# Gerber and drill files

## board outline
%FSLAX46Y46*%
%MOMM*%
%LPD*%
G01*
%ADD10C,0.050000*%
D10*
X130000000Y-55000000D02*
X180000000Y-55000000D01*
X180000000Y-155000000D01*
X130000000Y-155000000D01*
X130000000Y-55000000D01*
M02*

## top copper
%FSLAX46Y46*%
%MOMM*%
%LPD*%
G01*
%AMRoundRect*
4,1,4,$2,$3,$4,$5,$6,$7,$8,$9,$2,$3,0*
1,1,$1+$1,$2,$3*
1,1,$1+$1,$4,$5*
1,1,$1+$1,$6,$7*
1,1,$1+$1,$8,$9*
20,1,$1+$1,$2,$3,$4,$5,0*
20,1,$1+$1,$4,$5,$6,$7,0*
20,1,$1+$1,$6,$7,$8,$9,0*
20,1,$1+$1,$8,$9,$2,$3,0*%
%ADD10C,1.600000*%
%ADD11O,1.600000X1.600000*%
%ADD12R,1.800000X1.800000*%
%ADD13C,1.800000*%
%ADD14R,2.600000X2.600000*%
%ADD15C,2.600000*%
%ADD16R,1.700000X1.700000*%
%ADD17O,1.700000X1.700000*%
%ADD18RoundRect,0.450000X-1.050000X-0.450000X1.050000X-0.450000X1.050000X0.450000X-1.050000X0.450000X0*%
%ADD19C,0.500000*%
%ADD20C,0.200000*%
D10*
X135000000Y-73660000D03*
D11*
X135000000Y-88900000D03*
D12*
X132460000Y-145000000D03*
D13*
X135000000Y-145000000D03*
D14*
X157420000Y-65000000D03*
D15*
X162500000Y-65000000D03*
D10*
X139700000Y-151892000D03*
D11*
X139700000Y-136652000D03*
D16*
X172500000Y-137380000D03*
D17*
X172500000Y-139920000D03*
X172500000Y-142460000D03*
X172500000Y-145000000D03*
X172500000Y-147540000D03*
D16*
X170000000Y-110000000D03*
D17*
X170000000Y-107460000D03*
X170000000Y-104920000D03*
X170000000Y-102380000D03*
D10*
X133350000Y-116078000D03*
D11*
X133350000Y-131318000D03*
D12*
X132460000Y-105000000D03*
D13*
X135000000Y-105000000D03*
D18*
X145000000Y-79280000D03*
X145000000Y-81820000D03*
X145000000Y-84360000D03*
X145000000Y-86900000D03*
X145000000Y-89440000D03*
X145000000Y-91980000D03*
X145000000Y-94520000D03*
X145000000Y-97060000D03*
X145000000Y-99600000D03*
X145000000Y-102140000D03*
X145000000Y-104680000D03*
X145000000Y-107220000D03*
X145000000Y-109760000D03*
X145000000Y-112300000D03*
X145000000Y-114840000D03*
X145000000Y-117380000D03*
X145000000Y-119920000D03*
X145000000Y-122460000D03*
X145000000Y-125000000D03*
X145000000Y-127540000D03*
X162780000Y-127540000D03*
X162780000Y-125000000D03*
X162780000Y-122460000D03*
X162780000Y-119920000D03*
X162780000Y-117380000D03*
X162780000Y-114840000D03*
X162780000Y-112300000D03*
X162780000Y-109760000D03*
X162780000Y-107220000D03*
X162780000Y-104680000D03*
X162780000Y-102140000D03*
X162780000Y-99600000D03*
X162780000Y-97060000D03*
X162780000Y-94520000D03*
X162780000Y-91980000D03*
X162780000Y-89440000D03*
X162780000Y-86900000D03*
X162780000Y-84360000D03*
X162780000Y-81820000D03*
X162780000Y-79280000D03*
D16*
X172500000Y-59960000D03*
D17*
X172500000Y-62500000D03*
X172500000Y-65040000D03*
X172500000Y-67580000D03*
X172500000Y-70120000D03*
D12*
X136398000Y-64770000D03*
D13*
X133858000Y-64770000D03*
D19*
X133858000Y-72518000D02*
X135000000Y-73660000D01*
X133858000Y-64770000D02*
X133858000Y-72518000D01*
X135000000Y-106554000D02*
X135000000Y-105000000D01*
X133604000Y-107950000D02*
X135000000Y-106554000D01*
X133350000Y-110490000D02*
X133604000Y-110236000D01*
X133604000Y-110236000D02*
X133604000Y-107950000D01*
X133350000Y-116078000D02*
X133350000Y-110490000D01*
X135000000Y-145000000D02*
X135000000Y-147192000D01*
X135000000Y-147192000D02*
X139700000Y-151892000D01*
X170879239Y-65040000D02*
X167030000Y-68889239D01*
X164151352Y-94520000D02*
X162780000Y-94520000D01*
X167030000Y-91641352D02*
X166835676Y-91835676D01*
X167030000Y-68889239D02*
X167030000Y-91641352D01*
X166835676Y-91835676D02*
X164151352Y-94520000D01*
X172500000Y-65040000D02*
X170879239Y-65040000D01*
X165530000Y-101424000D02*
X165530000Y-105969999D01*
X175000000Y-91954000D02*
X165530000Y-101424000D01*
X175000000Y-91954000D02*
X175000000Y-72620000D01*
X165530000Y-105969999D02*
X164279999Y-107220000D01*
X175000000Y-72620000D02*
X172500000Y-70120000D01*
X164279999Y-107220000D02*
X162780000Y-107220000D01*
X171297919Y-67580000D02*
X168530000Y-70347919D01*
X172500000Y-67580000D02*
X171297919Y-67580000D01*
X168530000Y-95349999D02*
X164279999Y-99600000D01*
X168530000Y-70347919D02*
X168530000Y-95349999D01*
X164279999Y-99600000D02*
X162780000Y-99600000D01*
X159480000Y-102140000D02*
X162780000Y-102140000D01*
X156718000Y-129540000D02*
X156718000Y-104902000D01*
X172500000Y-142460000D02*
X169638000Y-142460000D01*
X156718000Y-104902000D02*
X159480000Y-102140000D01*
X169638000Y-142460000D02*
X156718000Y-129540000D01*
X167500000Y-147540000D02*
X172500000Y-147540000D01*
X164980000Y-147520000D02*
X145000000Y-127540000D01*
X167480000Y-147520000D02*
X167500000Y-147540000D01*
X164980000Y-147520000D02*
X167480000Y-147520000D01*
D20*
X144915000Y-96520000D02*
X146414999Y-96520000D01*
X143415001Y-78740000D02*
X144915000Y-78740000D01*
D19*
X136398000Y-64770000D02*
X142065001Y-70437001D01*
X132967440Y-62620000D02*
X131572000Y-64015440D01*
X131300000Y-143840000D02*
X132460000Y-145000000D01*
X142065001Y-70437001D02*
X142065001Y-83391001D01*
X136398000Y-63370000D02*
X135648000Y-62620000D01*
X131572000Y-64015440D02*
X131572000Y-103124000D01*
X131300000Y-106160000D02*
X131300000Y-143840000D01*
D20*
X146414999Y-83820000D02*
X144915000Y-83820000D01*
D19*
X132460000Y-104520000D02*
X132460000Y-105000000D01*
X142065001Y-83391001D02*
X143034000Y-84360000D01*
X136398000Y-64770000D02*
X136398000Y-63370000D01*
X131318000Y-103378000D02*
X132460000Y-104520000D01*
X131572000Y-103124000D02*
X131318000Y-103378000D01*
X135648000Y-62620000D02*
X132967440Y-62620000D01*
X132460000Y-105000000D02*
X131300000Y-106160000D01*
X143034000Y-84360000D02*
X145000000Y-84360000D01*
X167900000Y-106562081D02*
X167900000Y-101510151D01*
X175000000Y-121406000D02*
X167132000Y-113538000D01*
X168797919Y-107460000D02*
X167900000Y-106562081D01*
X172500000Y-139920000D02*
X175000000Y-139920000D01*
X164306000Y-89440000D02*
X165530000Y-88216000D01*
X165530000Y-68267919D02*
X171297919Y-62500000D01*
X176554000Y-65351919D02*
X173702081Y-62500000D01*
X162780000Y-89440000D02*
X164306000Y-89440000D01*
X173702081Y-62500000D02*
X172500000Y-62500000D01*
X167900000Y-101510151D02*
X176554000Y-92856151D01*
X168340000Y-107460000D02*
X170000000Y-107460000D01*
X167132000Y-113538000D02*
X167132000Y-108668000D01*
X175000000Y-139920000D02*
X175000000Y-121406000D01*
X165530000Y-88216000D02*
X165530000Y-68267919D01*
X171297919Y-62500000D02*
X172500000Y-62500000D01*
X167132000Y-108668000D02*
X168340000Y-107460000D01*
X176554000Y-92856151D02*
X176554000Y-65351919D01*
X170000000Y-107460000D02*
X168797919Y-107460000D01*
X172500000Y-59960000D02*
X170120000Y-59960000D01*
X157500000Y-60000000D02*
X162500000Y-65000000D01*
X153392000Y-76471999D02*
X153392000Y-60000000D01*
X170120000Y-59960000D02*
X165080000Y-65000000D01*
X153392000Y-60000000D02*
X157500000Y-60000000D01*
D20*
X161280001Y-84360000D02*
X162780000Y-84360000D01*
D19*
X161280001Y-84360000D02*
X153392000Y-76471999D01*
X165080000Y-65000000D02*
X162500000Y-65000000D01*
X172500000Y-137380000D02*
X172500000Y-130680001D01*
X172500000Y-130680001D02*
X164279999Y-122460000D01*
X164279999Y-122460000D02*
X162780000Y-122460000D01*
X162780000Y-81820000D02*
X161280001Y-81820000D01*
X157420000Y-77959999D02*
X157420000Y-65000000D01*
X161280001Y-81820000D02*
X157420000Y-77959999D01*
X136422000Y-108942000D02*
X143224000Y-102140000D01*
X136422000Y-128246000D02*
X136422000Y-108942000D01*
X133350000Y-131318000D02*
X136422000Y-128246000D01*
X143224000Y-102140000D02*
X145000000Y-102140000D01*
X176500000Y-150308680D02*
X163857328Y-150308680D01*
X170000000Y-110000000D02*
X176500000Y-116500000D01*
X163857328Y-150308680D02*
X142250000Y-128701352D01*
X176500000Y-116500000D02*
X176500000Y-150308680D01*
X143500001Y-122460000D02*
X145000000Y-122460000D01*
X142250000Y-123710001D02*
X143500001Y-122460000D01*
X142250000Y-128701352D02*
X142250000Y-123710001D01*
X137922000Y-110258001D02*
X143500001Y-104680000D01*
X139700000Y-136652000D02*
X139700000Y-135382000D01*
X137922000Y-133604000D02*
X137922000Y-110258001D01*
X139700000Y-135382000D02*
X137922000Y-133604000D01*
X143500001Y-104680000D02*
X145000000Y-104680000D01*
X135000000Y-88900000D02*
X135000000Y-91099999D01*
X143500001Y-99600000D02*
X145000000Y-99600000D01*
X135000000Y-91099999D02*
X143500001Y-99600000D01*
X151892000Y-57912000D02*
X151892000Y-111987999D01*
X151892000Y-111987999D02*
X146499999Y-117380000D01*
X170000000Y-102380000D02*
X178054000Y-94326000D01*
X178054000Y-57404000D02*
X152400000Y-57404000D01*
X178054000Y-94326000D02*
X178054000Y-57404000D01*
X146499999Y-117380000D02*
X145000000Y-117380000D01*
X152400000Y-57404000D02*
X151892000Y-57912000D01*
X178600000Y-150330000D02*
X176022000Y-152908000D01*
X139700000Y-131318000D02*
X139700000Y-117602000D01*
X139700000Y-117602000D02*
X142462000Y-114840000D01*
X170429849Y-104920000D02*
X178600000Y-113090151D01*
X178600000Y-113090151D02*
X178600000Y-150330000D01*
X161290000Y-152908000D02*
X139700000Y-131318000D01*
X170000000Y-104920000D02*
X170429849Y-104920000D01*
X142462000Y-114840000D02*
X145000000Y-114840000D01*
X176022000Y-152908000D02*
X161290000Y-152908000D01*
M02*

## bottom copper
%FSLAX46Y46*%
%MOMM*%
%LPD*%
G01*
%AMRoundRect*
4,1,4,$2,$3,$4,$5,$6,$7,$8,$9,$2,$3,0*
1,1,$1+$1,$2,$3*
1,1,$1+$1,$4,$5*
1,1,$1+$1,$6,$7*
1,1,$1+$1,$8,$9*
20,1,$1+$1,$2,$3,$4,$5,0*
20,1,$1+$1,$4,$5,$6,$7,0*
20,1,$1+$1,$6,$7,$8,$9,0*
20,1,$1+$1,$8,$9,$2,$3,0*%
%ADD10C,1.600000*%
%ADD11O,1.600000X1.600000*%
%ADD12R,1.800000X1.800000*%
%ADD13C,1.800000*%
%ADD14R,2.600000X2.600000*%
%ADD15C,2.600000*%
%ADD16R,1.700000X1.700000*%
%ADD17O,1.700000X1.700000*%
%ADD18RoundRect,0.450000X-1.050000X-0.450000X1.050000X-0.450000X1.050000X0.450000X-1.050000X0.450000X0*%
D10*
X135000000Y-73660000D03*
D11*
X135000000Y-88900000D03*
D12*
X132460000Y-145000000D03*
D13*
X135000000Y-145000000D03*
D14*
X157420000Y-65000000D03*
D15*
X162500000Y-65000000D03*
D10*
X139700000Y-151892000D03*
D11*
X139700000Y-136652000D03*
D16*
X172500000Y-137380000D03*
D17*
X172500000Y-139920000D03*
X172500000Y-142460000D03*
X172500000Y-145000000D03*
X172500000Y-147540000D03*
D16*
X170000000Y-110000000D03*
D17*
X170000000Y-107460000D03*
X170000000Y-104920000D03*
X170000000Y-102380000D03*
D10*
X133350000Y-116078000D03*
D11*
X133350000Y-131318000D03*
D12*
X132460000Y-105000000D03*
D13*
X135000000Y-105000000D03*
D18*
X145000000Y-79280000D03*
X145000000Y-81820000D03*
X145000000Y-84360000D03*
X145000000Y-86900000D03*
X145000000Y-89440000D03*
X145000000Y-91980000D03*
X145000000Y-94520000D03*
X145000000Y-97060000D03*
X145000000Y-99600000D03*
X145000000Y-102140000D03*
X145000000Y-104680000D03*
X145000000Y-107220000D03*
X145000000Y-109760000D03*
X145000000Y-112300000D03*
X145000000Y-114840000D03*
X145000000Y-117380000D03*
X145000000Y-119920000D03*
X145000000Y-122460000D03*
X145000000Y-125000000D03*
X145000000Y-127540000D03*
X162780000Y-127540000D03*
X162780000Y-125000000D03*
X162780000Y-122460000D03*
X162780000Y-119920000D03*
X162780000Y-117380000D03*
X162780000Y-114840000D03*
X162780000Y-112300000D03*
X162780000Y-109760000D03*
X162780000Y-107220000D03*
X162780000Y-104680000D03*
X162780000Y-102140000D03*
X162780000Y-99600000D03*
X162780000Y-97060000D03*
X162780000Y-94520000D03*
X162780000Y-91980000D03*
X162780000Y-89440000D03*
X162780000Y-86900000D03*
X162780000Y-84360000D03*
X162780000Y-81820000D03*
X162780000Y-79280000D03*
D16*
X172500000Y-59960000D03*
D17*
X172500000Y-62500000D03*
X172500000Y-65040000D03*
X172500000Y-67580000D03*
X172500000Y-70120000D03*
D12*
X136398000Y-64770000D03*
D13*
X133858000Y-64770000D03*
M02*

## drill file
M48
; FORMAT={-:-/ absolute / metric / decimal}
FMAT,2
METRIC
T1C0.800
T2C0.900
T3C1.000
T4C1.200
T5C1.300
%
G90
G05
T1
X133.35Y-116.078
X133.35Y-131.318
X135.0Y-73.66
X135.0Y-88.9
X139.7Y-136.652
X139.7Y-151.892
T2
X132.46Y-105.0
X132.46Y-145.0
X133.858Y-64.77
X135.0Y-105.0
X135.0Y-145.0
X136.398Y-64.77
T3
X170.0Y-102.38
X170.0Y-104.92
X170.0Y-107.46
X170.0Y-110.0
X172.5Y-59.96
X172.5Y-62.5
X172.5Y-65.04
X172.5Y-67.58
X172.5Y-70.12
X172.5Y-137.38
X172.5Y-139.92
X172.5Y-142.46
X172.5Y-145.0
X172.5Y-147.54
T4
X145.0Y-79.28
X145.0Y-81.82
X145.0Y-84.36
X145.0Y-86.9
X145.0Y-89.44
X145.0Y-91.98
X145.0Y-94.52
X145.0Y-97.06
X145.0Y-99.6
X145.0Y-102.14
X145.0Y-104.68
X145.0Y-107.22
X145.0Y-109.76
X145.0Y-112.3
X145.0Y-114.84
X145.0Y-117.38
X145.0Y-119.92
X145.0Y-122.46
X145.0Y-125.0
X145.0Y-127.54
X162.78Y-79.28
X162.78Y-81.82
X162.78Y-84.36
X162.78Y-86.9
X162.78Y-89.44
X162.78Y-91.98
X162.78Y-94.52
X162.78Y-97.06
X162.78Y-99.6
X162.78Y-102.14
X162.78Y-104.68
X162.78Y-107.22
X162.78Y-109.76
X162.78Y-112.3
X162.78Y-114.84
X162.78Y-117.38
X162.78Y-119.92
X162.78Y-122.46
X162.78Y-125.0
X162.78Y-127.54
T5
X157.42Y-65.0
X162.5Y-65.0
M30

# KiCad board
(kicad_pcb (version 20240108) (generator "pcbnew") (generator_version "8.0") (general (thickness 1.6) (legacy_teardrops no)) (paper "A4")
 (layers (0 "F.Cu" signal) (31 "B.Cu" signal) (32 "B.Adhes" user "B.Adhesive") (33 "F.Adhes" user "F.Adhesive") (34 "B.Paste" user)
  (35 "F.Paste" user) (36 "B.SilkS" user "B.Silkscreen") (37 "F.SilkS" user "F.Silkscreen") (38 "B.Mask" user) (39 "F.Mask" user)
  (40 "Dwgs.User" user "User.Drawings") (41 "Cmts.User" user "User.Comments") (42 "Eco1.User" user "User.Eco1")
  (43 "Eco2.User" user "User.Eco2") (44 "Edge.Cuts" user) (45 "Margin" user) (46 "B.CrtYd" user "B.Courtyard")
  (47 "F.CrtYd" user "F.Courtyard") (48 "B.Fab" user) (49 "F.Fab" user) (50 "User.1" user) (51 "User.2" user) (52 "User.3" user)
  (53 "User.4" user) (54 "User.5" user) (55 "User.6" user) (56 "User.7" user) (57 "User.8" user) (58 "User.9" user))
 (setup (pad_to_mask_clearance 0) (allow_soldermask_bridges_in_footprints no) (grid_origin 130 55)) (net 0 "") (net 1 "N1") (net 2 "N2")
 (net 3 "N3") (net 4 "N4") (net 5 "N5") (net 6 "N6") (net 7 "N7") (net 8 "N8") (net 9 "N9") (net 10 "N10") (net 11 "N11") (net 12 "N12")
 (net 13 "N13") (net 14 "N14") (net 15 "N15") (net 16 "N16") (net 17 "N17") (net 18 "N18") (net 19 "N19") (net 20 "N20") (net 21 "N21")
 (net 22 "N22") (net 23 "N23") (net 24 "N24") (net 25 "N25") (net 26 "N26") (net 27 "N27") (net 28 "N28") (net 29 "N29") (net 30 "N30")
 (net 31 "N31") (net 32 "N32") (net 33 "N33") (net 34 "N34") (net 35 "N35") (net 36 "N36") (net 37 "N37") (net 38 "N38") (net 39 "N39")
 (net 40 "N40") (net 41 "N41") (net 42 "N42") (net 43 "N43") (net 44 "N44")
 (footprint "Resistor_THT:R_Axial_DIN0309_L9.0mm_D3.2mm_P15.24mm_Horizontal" (layer "F.Cu") (at 135 73.66 -90)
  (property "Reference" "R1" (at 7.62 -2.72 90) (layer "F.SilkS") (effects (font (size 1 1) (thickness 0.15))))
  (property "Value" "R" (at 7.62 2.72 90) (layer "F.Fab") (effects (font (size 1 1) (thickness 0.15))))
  (pad "1" thru_hole circle (at 0 0 270) (size 1.6 1.6) (drill 0.8) (layers "*.Cu" "*.Mask") (remove_unused_layers no) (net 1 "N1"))
  (pad "2" thru_hole oval (at 15.24 0 270) (size 1.6 1.6) (drill 0.8) (layers "*.Cu" "*.Mask") (remove_unused_layers no) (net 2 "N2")))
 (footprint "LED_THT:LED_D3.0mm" (layer "F.Cu") (at 132.46 145)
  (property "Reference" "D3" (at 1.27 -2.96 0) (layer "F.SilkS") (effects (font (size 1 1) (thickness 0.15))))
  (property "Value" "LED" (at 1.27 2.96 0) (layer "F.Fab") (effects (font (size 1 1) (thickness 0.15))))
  (pad "1" thru_hole rect (at 0 0) (size 1.8 1.8) (drill 0.9) (layers "*.Cu" "*.Mask") (remove_unused_layers no) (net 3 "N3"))
  (pad "2" thru_hole circle (at 2.54 0) (size 1.8 1.8) (drill 0.9) (layers "*.Cu" "*.Mask") (remove_unused_layers no) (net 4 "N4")))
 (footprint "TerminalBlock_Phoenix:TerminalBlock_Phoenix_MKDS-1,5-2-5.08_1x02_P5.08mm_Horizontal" (layer "F.Cu") (at 157.42 65)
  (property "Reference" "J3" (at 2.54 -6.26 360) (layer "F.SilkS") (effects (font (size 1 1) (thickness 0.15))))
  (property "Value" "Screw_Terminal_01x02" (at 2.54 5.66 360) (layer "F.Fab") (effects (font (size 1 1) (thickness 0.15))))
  (pad "1" thru_hole rect (at 0 0) (size 2.6 2.6) (drill 1.3) (layers "*.Cu" "*.Mask") (remove_unused_layers no) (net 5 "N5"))
  (pad "2" thru_hole circle (at 5.08 0) (size 2.6 2.6) (drill 1.3) (layers "*.Cu" "*.Mask") (remove_unused_layers no) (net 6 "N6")))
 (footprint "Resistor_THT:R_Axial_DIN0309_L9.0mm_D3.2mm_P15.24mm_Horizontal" (layer "F.Cu") (at 139.7 151.892 90)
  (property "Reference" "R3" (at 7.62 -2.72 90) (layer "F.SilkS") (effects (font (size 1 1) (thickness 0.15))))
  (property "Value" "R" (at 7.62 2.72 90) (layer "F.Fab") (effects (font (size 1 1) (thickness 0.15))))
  (pad "1" thru_hole circle (at 0 0 90) (size 1.6 1.6) (drill 0.8) (layers "*.Cu" "*.Mask") (remove_unused_layers no) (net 4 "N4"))
  (pad "2" thru_hole oval (at 15.24 0 90) (size 1.6 1.6) (drill 0.8) (layers "*.Cu" "*.Mask") (remove_unused_layers no) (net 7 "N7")))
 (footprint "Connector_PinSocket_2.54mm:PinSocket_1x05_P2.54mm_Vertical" (layer "F.Cu") (at 172.5 137.38)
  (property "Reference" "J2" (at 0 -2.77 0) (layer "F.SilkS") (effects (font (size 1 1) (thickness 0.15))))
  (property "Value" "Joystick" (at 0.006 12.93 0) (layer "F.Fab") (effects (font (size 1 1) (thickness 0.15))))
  (pad "1" thru_hole rect (at 0 0) (size 1.7 1.7) (drill 1) (layers "*.Cu" "*.Mask") (remove_unused_layers no) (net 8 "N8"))
  (pad "2" thru_hole oval (at 0 2.54) (size 1.7 1.7) (drill 1) (layers "*.Cu" "*.Mask") (remove_unused_layers no) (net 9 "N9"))
  (pad "3" thru_hole oval (at 0 5.08) (size 1.7 1.7) (drill 1) (layers "*.Cu" "*.Mask") (remove_unused_layers no) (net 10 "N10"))
  (pad "4" thru_hole oval (at 0 7.62) (size 1.7 1.7) (drill 1) (layers "*.Cu" "*.Mask") (remove_unused_layers no) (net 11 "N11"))
  (pad "5" thru_hole oval (at 0 10.16) (size 1.7 1.7) (drill 1) (layers "*.Cu" "*.Mask") (remove_unused_layers no) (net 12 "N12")))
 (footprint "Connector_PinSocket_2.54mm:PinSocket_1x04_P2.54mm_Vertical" (layer "F.Cu") (at 170 110 180)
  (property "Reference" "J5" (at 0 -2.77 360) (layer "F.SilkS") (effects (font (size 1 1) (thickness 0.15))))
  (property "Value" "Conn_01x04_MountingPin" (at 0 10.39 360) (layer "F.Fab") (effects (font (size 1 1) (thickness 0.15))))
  (pad "1" thru_hole rect (at 0 0 180) (size 1.7 1.7) (drill 1) (layers "*.Cu" "*.Mask") (remove_unused_layers no) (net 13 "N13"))
  (pad "2" thru_hole oval (at 0 2.54 180) (size 1.7 1.7) (drill 1) (layers "*.Cu" "*.Mask") (remove_unused_layers no) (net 9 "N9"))
  (pad "3" thru_hole oval (at 0 5.08 180) (size 1.7 1.7) (drill 1) (layers "*.Cu" "*.Mask") (remove_unused_layers no) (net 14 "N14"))
  (pad "4" thru_hole oval (at 0 7.62 180) (size 1.7 1.7) (drill 1) (layers "*.Cu" "*.Mask") (remove_unused_layers no) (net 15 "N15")))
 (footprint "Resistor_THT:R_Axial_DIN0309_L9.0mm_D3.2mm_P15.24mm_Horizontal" (layer "F.Cu") (at 133.35 116.078 -90)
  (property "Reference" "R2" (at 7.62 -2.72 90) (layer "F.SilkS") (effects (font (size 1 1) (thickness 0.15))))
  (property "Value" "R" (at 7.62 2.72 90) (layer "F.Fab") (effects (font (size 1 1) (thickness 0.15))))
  (pad "1" thru_hole circle (at 0 0 270) (size 1.6 1.6) (drill 0.8) (layers "*.Cu" "*.Mask") (remove_unused_layers no) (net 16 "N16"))
  (pad "2" thru_hole oval (at 15.24 0 270) (size 1.6 1.6) (drill 0.8) (layers "*.Cu" "*.Mask") (remove_unused_layers no) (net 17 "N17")))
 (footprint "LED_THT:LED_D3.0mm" (layer "F.Cu") (at 132.46 105)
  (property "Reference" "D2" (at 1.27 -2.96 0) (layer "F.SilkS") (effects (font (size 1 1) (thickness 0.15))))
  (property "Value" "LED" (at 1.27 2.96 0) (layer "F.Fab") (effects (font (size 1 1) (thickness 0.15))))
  (pad "1" thru_hole rect (at 0 0) (size 1.8 1.8) (drill 0.9) (layers "*.Cu" "*.Mask") (remove_unused_layers no) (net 3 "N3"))
  (pad "2" thru_hole circle (at 2.54 0) (size 1.8 1.8) (drill 0.9) (layers "*.Cu" "*.Mask") (remove_unused_layers no) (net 16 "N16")))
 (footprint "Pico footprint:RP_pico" (layer "F.Cu") (at 153.89 103.41)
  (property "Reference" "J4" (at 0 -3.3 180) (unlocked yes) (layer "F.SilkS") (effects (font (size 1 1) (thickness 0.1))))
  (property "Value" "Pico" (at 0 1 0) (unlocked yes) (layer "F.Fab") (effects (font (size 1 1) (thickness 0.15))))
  (pad "1" thru_hole roundrect (at -8.89 -24.13) (size 3 1.8) (drill 1.2) (layers "*.Cu" "*.Mask") (remove_unused_layers no)
   (roundrect_rratio 0.25) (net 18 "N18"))
  (pad "2" thru_hole roundrect (at -8.89 -21.59) (size 3 1.8) (drill 1.2) (layers "*.Cu" "*.Mask") (remove_unused_layers no)
   (roundrect_rratio 0.25) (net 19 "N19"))
  (pad "3" thru_hole roundrect (at -8.89 -19.05) (size 3 1.8) (drill 1.2) (layers "*.Cu" "*.Mask") (remove_unused_layers no)
   (roundrect_rratio 0.25) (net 3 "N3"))
  (pad "4" thru_hole roundrect (at -8.89 -16.51) (size 3 1.8) (drill 1.2) (layers "*.Cu" "*.Mask") (remove_unused_layers no)
   (roundrect_rratio 0.25) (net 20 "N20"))
  (pad "5" thru_hole roundrect (at -8.89 -13.97) (size 3 1.8) (drill 1.2) (layers "*.Cu" "*.Mask") (remove_unused_layers no)
   (roundrect_rratio 0.25) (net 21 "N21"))
  (pad "6" thru_hole roundrect (at -8.89 -11.43) (size 3 1.8) (drill 1.2) (layers "*.Cu" "*.Mask") (remove_unused_layers no)
   (roundrect_rratio 0.25) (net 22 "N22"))
  (pad "7" thru_hole roundrect (at -8.89 -8.89) (size 3 1.8) (drill 1.2) (layers "*.Cu" "*.Mask") (remove_unused_layers no)
   (roundrect_rratio 0.25) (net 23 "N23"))
  (pad "8" thru_hole roundrect (at -8.89 -6.35) (size 3 1.8) (drill 1.2) (layers "*.Cu" "*.Mask") (remove_unused_layers no)
   (roundrect_rratio 0.25) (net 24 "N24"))
  (pad "9" thru_hole roundrect (at -8.89 -3.81) (size 3 1.8) (drill 1.2) (layers "*.Cu" "*.Mask") (remove_unused_layers no)
   (roundrect_rratio 0.25) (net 2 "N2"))
  (pad "10" thru_hole roundrect (at -8.89 -1.27) (size 3 1.8) (drill 1.2) (layers "*.Cu" "*.Mask") (remove_unused_layers no)
   (roundrect_rratio 0.25) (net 17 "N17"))
  (pad "11" thru_hole roundrect (at -8.89 1.27) (size 3 1.8) (drill 1.2) (layers "*.Cu" "*.Mask") (remove_unused_layers no)
   (roundrect_rratio 0.25) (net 7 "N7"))
  (pad "12" thru_hole roundrect (at -8.89 3.81) (size 3 1.8) (drill 1.2) (layers "*.Cu" "*.Mask") (remove_unused_layers no)
   (roundrect_rratio 0.25) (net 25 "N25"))
  (pad "13" thru_hole roundrect (at -8.89 6.35) (size 3 1.8) (drill 1.2) (layers "*.Cu" "*.Mask") (remove_unused_layers no)
   (roundrect_rratio 0.25) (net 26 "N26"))
  (pad "14" thru_hole roundrect (at -8.89 8.89) (size 3 1.8) (drill 1.2) (layers "*.Cu" "*.Mask") (remove_unused_layers no)
   (roundrect_rratio 0.25) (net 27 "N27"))
  (pad "15" thru_hole roundrect (at -8.89 11.43) (size 3 1.8) (drill 1.2) (layers "*.Cu" "*.Mask") (remove_unused_layers no)
   (roundrect_rratio 0.25) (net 14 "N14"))
  (pad "16" thru_hole roundrect (at -8.89 13.97) (size 3 1.8) (drill 1.2) (layers "*.Cu" "*.Mask") (remove_unused_layers no)
   (roundrect_rratio 0.25) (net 15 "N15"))
  (pad "17" thru_hole roundrect (at -8.89 16.51) (size 3 1.8) (drill 1.2) (layers "*.Cu" "*.Mask") (remove_unused_layers no)
   (roundrect_rratio 0.25) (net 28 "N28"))
  (pad "18" thru_hole roundrect (at -8.89 19.05) (size 3 1.8) (drill 1.2) (layers "*.Cu" "*.Mask") (remove_unused_layers no)
   (roundrect_rratio 0.25) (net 13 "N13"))
  (pad "19" thru_hole roundrect (at -8.89 21.59) (size 3 1.8) (drill 1.2) (layers "*.Cu" "*.Mask") (remove_unused_layers no)
   (roundrect_rratio 0.25) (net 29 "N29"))
  (pad "20" thru_hole roundrect (at -8.89 24.13) (size 3 1.8) (drill 1.2) (layers "*.Cu" "*.Mask") (remove_unused_layers no)
   (roundrect_rratio 0.25) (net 12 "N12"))
  (pad "21" thru_hole roundrect (at 8.89 24.13) (size 3 1.8) (drill 1.2) (layers "*.Cu" "*.Mask") (remove_unused_layers no)
   (roundrect_rratio 0.25) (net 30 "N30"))
  (pad "22" thru_hole roundrect (at 8.89 21.59) (size 3 1.8) (drill 1.2) (layers "*.Cu" "*.Mask") (remove_unused_layers no)
   (roundrect_rratio 0.25) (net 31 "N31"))
  (pad "23" thru_hole roundrect (at 8.89 19.05) (size 3 1.8) (drill 1.2) (layers "*.Cu" "*.Mask") (remove_unused_layers no)
   (roundrect_rratio 0.25) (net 8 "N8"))
  (pad "24" thru_hole roundrect (at 8.89 16.51) (size 3 1.8) (drill 1.2) (layers "*.Cu" "*.Mask") (remove_unused_layers no)
   (roundrect_rratio 0.25) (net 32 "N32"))
  (pad "25" thru_hole roundrect (at 8.89 13.97) (size 3 1.8) (drill 1.2) (layers "*.Cu" "*.Mask") (remove_unused_layers no)
   (roundrect_rratio 0.25) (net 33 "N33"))
  (pad "26" thru_hole roundrect (at 8.89 11.43) (size 3 1.8) (drill 1.2) (layers "*.Cu" "*.Mask") (remove_unused_layers no)
   (roundrect_rratio 0.25) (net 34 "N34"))
  (pad "27" thru_hole roundrect (at 8.89 8.89) (size 3 1.8) (drill 1.2) (layers "*.Cu" "*.Mask") (remove_unused_layers no)
   (roundrect_rratio 0.25) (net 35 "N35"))
  (pad "28" thru_hole roundrect (at 8.89 6.35) (size 3 1.8) (drill 1.2) (layers "*.Cu" "*.Mask") (remove_unused_layers no)
   (roundrect_rratio 0.25) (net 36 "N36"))
  (pad "29" thru_hole roundrect (at 8.89 3.81) (size 3 1.8) (drill 1.2) (layers "*.Cu" "*.Mask") (remove_unused_layers no)
   (roundrect_rratio 0.25) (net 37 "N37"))
  (pad "30" thru_hole roundrect (at 8.89 1.27) (size 3 1.8) (drill 1.2) (layers "*.Cu" "*.Mask") (remove_unused_layers no)
   (roundrect_rratio 0.25) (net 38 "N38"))
  (pad "31" thru_hole roundrect (at 8.89 -1.27) (size 3 1.8) (drill 1.2) (layers "*.Cu" "*.Mask") (remove_unused_layers no)
   (roundrect_rratio 0.25) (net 10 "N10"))
  (pad "32" thru_hole roundrect (at 8.89 -3.81) (size 3 1.8) (drill 1.2) (layers "*.Cu" "*.Mask") (remove_unused_layers no)
   (roundrect_rratio 0.25) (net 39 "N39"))
  (pad "33" thru_hole roundrect (at 8.89 -6.35) (size 3 1.8) (drill 1.2) (layers "*.Cu" "*.Mask") (remove_unused_layers no)
   (roundrect_rratio 0.25) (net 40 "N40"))
  (pad "34" thru_hole roundrect (at 8.89 -8.89) (size 3 1.8) (drill 1.2) (layers "*.Cu" "*.Mask") (remove_unused_layers no)
   (roundrect_rratio 0.25) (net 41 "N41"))
  (pad "35" thru_hole roundrect (at 8.89 -11.43) (size 3 1.8) (drill 1.2) (layers "*.Cu" "*.Mask") (remove_unused_layers no)
   (roundrect_rratio 0.25) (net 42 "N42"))
  (pad "36" thru_hole roundrect (at 8.89 -13.97) (size 3 1.8) (drill 1.2) (layers "*.Cu" "*.Mask") (remove_unused_layers no)
   (roundrect_rratio 0.25) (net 9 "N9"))
  (pad "37" thru_hole roundrect (at 8.89 -16.51) (size 3 1.8) (drill 1.2) (layers "*.Cu" "*.Mask") (remove_unused_layers no)
   (roundrect_rratio 0.25) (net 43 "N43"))
  (pad "38" thru_hole roundrect (at 8.89 -19.05) (size 3 1.8) (drill 1.2) (layers "*.Cu" "*.Mask") (remove_unused_layers no)
   (roundrect_rratio 0.25) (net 6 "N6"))
  (pad "39" thru_hole roundrect (at 8.89 -21.59) (size 3 1.8) (drill 1.2) (layers "*.Cu" "*.Mask") (remove_unused_layers no)
   (roundrect_rratio 0.25) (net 5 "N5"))
  (pad "40" thru_hole roundrect (at 8.89 -24.13) (size 3 1.8) (drill 1.2) (layers "*.Cu" "*.Mask") (remove_unused_layers no)
   (roundrect_rratio 0.25) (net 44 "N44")))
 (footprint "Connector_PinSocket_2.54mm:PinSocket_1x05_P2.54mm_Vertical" (layer "F.Cu") (at 172.5 59.96)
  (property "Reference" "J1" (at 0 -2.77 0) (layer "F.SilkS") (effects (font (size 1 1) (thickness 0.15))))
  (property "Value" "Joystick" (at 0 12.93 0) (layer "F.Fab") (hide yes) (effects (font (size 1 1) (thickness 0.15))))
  (pad "1" thru_hole rect (at 0 0) (size 1.7 1.7) (drill 1) (layers "*.Cu" "*.Mask") (remove_unused_layers no) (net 6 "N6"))
  (pad "2" thru_hole oval (at 0 2.54) (size 1.7 1.7) (drill 1) (layers "*.Cu" "*.Mask") (remove_unused_layers no) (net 9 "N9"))
  (pad "3" thru_hole oval (at 0 5.08) (size 1.7 1.7) (drill 1) (layers "*.Cu" "*.Mask") (remove_unused_layers no) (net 41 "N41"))
  (pad "4" thru_hole oval (at 0 7.62) (size 1.7 1.7) (drill 1) (layers "*.Cu" "*.Mask") (remove_unused_layers no) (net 39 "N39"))
  (pad "5" thru_hole oval (at 0 10.16) (size 1.7 1.7) (drill 1) (layers "*.Cu" "*.Mask") (remove_unused_layers no) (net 37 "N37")))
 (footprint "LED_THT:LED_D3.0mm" (layer "F.Cu") (at 136.398 64.77 180)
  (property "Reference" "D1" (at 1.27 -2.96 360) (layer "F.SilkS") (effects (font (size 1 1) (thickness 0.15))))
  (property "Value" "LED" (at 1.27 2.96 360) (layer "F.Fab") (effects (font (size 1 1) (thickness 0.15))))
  (pad "1" thru_hole rect (at 0 0 180) (size 1.8 1.8) (drill 0.9) (layers "*.Cu" "*.Mask") (remove_unused_layers no) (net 3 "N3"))
  (pad "2" thru_hole circle (at 2.54 0 180) (size 1.8 1.8) (drill 0.9) (layers "*.Cu" "*.Mask") (remove_unused_layers no) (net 1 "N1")))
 (gr_rect (start 130 55) (end 180 155) (stroke (width 0.05) (type default)) (fill none) (layer "Edge.Cuts"))
 (segment (start 133.858 72.518) (end 135 73.66) (width 0.5) (layer "F.Cu") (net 1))
 (segment (start 133.858 64.77) (end 133.858 72.518) (width 0.5) (layer "F.Cu") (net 1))
 (segment (start 135 106.554) (end 135 105) (width 0.5) (layer "F.Cu") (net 16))
 (segment (start 133.604 107.95) (end 135 106.554) (width 0.5) (layer "F.Cu") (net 16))
 (segment (start 133.35 110.49) (end 133.604 110.236) (width 0.5) (layer "F.Cu") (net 16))
 (segment (start 133.604 110.236) (end 133.604 107.95) (width 0.5) (layer "F.Cu") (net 16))
 (segment (start 133.35 116.078) (end 133.35 110.49) (width 0.5) (layer "F.Cu") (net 16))
 (segment (start 135 145) (end 135 147.192) (width 0.5) (layer "F.Cu") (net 4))
 (segment (start 135 147.192) (end 139.7 151.892) (width 0.5) (layer "F.Cu") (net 4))
 (segment (start 170.879239 65.04) (end 167.03 68.889239) (width 0.5) (layer "F.Cu") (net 41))
 (segment (start 164.151352 94.52) (end 162.78 94.52) (width 0.5) (layer "F.Cu") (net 41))
 (segment (start 167.03 91.641352) (end 166.835676 91.835676) (width 0.5) (layer "F.Cu") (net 41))
 (segment (start 167.03 68.889239) (end 167.03 91.641352) (width 0.5) (layer "F.Cu") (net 41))
 (segment (start 166.835676 91.835676) (end 164.151352 94.52) (width 0.5) (layer "F.Cu") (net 41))
 (segment (start 172.5 65.04) (end 170.879239 65.04) (width 0.5) (layer "F.Cu") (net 41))
 (segment (start 165.53 101.424) (end 165.53 105.969999) (width 0.5) (layer "F.Cu") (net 37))
 (segment (start 175 91.954) (end 165.53 101.424) (width 0.5) (layer "F.Cu") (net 37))
 (segment (start 175 91.954) (end 175 72.62) (width 0.5) (layer "F.Cu") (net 37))
 (segment (start 165.53 105.969999) (end 164.279999 107.22) (width 0.5) (layer "F.Cu") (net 37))
 (segment (start 175 72.62) (end 172.5 70.12) (width 0.5) (layer "F.Cu") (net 37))
 (segment (start 164.279999 107.22) (end 162.78 107.22) (width 0.5) (layer "F.Cu") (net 37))
 (segment (start 171.297919 67.58) (end 168.53 70.347919) (width 0.5) (layer "F.Cu") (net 39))
 (segment (start 172.5 67.58) (end 171.297919 67.58) (width 0.5) (layer "F.Cu") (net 39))
 (segment (start 168.53 95.349999) (end 164.279999 99.6) (width 0.5) (layer "F.Cu") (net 39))
 (segment (start 168.53 70.347919) (end 168.53 95.349999) (width 0.5) (layer "F.Cu") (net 39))
 (segment (start 164.279999 99.6) (end 162.78 99.6) (width 0.5) (layer "F.Cu") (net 39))
 (segment (start 159.48 102.14) (end 162.78 102.14) (width 0.5) (layer "F.Cu") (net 10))
 (segment (start 156.718 129.54) (end 156.718 104.902) (width 0.5) (layer "F.Cu") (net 10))
 (segment (start 172.5 142.46) (end 169.638 142.46) (width 0.5) (layer "F.Cu") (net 10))
 (segment (start 156.718 104.902) (end 159.48 102.14) (width 0.5) (layer "F.Cu") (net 10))
 (segment (start 169.638 142.46) (end 156.718 129.54) (width 0.5) (layer "F.Cu") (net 10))
 (segment (start 167.5 147.54) (end 172.5 147.54) (width 0.5) (layer "F.Cu") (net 12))
 (segment (start 164.98 147.52) (end 145 127.54) (width 0.5) (layer "F.Cu") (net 12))
 (segment (start 167.48 147.52) (end 167.5 147.54) (width 0.5) (layer "F.Cu") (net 12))
 (segment (start 164.98 147.52) (end 167.48 147.52) (width 0.5) (layer "F.Cu") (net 12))
 (segment (start 144.915 96.52) (end 146.414999 96.52) (width 0.2) (layer "F.Cu") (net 24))
 (segment (start 143.415001 78.74) (end 144.915 78.74) (width 0.2) (layer "F.Cu") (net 18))
 (segment (start 136.398 64.77) (end 142.065001 70.437001) (width 0.5) (layer "F.Cu") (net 3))
 (segment (start 132.96744 62.62) (end 131.572 64.01544) (width 0.5) (layer "F.Cu") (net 3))
 (segment (start 131.3 143.84) (end 132.46 145) (width 0.5) (layer "F.Cu") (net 3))
 (segment (start 142.065001 70.437001) (end 142.065001 83.391001) (width 0.5) (layer "F.Cu") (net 3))
 (segment (start 136.398 63.37) (end 135.648 62.62) (width 0.5) (layer "F.Cu") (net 3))
 (segment (start 131.572 64.01544) (end 131.572 103.124) (width 0.5) (layer "F.Cu") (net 3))
 (segment (start 131.3 106.16) (end 131.3 143.84) (width 0.5) (layer "F.Cu") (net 3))
 (segment (start 146.414999 83.82) (end 144.915 83.82) (width 0.2) (layer "F.Cu") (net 3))
 (segment (start 132.46 104.52) (end 132.46 105) (width 0.5) (layer "F.Cu") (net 3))
 (segment (start 142.065001 83.391001) (end 143.034 84.36) (width 0.5) (layer "F.Cu") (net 3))
 (segment (start 136.398 64.77) (end 136.398 63.37) (width 0.5) (layer "F.Cu") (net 3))
 (segment (start 131.318 103.378) (end 132.46 104.52) (width 0.5) (layer "F.Cu") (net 3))
 (segment (start 131.572 103.124) (end 131.318 103.378) (width 0.5) (layer "F.Cu") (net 3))
 (segment (start 135.648 62.62) (end 132.96744 62.62) (width 0.5) (layer "F.Cu") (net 3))
 (segment (start 132.46 105) (end 131.3 106.16) (width 0.5) (layer "F.Cu") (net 3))
 (segment (start 143.034 84.36) (end 145 84.36) (width 0.5) (layer "F.Cu") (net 3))
 (segment (start 167.9 106.562081) (end 167.9 101.510151) (width 0.5) (layer "F.Cu") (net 9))
 (segment (start 175 121.406) (end 167.132 113.538) (width 0.5) (layer "F.Cu") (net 9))
 (segment (start 168.797919 107.46) (end 167.9 106.562081) (width 0.5) (layer "F.Cu") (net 9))
 (segment (start 172.5 139.92) (end 175 139.92) (width 0.5) (layer "F.Cu") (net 9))
 (segment (start 164.306 89.44) (end 165.53 88.216) (width 0.5) (layer "F.Cu") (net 9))
 (segment (start 165.53 68.267919) (end 171.297919 62.5) (width 0.5) (layer "F.Cu") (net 9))
 (segment (start 176.554 65.351919) (end 173.702081 62.5) (width 0.5) (layer "F.Cu") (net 9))
 (segment (start 162.78 89.44) (end 164.306 89.44) (width 0.5) (layer "F.Cu") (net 9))
 (segment (start 173.702081 62.5) (end 172.5 62.5) (width 0.5) (layer "F.Cu") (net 9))
 (segment (start 167.9 101.510151) (end 176.554 92.856151) (width 0.5) (layer "F.Cu") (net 9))
 (segment (start 168.34 107.46) (end 170 107.46) (width 0.5) (layer "F.Cu") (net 9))
 (segment (start 167.132 113.538) (end 167.132 108.668) (width 0.5) (layer "F.Cu") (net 9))
 (segment (start 175 139.92) (end 175 121.406) (width 0.5) (layer "F.Cu") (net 9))
 (segment (start 165.53 88.216) (end 165.53 68.267919) (width 0.5) (layer "F.Cu") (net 9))
 (segment (start 171.297919 62.5) (end 172.5 62.5) (width 0.5) (layer "F.Cu") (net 9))
 (segment (start 167.132 108.668) (end 168.34 107.46) (width 0.5) (layer "F.Cu") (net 9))
 (segment (start 176.554 92.856151) (end 176.554 65.351919) (width 0.5) (layer "F.Cu") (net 9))
 (segment (start 170 107.46) (end 168.797919 107.46) (width 0.5) (layer "F.Cu") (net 9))
 (segment (start 172.5 59.96) (end 170.12 59.96) (width 0.5) (layer "F.Cu") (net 6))
 (segment (start 157.5 60) (end 162.5 65) (width 0.5) (layer "F.Cu") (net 6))
 (segment (start 153.392 76.471999) (end 153.392 60) (width 0.5) (layer "F.Cu") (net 6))
 (segment (start 170.12 59.96) (end 165.08 65) (width 0.5) (layer "F.Cu") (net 6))
 (segment (start 153.392 60) (end 157.5 60) (width 0.5) (layer "F.Cu") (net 6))
 (segment (start 161.280001 84.36) (end 162.78 84.36) (width 0.2) (layer "F.Cu") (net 6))
 (segment (start 161.280001 84.36) (end 153.392 76.471999) (width 0.5) (layer "F.Cu") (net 6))
 (segment (start 165.08 65) (end 162.5 65) (width 0.5) (layer "F.Cu") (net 6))
 (segment (start 172.5 137.38) (end 172.5 130.680001) (width 0.5) (layer "F.Cu") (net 8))
 (segment (start 172.5 130.680001) (end 164.279999 122.46) (width 0.5) (layer "F.Cu") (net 8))
 (segment (start 164.279999 122.46) (end 162.78 122.46) (width 0.5) (layer "F.Cu") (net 8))
 (segment (start 162.78 81.82) (end 161.280001 81.82) (width 0.5) (layer "F.Cu") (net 5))
 (segment (start 157.42 77.959999) (end 157.42 65) (width 0.5) (layer "F.Cu") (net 5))
 (segment (start 161.280001 81.82) (end 157.42 77.959999) (width 0.5) (layer "F.Cu") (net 5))
 (segment (start 136.422 108.942) (end 143.224 102.14) (width 0.5) (layer "F.Cu") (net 17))
 (segment (start 136.422 128.246) (end 136.422 108.942) (width 0.5) (layer "F.Cu") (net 17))
 (segment (start 133.35 131.318) (end 136.422 128.246) (width 0.5) (layer "F.Cu") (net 17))
 (segment (start 143.224 102.14) (end 145 102.14) (width 0.5) (layer "F.Cu") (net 17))
 (segment (start 176.5 150.30868) (end 163.857328 150.30868) (width 0.5) (layer "F.Cu") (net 13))
 (segment (start 170 110) (end 176.5 116.5) (width 0.5) (layer "F.Cu") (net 13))
 (segment (start 163.857328 150.30868) (end 142.25 128.701352) (width 0.5) (layer "F.Cu") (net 13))
 (segment (start 176.5 116.5) (end 176.5 150.30868) (width 0.5) (layer "F.Cu") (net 13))
 (segment (start 143.500001 122.46) (end 145 122.46) (width 0.5) (layer "F.Cu") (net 13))
 (segment (start 142.25 123.710001) (end 143.500001 122.46) (width 0.5) (layer "F.Cu") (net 13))
 (segment (start 142.25 128.701352) (end 142.25 123.710001) (width 0.5) (layer "F.Cu") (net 13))
 (segment (start 137.922 110.258001) (end 143.500001 104.68) (width 0.5) (layer "F.Cu") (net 7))
 (segment (start 139.7 136.652) (end 139.7 135.382) (width 0.5) (layer "F.Cu") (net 7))
 (segment (start 137.922 133.604) (end 137.922 110.258001) (width 0.5) (layer "F.Cu") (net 7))
 (segment (start 139.7 135.382) (end 137.922 133.604) (width 0.5) (layer "F.Cu") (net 7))
 (segment (start 143.500001 104.68) (end 145 104.68) (width 0.5) (layer "F.Cu") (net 7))
 (segment (start 135 88.9) (end 135 91.099999) (width 0.5) (layer "F.Cu") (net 2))
 (segment (start 143.500001 99.6) (end 145 99.6) (width 0.5) (layer "F.Cu") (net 2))
 (segment (start 135 91.099999) (end 143.500001 99.6) (width 0.5) (layer "F.Cu") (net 2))
 (segment (start 151.892 57.912) (end 151.892 111.987999) (width 0.5) (layer "F.Cu") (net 15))
 (segment (start 151.892 111.987999) (end 146.499999 117.38) (width 0.5) (layer "F.Cu") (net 15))
 (segment (start 170 102.38) (end 178.054 94.326) (width 0.5) (layer "F.Cu") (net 15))
 (segment (start 178.054 57.404) (end 152.4 57.404) (width 0.5) (layer "F.Cu") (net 15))
 (segment (start 178.054 94.326) (end 178.054 57.404) (width 0.5) (layer "F.Cu") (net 15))
 (segment (start 146.499999 117.38) (end 145 117.38) (width 0.5) (layer "F.Cu") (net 15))
 (segment (start 152.4 57.404) (end 151.892 57.912) (width 0.5) (layer "F.Cu") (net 15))
 (segment (start 178.6 150.33) (end 176.022 152.908) (width 0.5) (layer "F.Cu") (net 14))
 (segment (start 139.7 131.318) (end 139.7 117.602) (width 0.5) (layer "F.Cu") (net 14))
 (segment (start 139.7 117.602) (end 142.462 114.84) (width 0.5) (layer "F.Cu") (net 14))
 (segment (start 170.429849 104.92) (end 178.6 113.090151) (width 0.5) (layer "F.Cu") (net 14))
 (segment (start 178.6 113.090151) (end 178.6 150.33) (width 0.5) (layer "F.Cu") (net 14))
 (segment (start 161.29 152.908) (end 139.7 131.318) (width 0.5) (layer "F.Cu") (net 14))
 (segment (start 170 104.92) (end 170.429849 104.92) (width 0.5) (layer "F.Cu") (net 14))
 (segment (start 142.462 114.84) (end 145 114.84) (width 0.5) (layer "F.Cu") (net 14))
 (segment (start 176.022 152.908) (end 161.29 152.908) (width 0.5) (layer "F.Cu") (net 14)))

